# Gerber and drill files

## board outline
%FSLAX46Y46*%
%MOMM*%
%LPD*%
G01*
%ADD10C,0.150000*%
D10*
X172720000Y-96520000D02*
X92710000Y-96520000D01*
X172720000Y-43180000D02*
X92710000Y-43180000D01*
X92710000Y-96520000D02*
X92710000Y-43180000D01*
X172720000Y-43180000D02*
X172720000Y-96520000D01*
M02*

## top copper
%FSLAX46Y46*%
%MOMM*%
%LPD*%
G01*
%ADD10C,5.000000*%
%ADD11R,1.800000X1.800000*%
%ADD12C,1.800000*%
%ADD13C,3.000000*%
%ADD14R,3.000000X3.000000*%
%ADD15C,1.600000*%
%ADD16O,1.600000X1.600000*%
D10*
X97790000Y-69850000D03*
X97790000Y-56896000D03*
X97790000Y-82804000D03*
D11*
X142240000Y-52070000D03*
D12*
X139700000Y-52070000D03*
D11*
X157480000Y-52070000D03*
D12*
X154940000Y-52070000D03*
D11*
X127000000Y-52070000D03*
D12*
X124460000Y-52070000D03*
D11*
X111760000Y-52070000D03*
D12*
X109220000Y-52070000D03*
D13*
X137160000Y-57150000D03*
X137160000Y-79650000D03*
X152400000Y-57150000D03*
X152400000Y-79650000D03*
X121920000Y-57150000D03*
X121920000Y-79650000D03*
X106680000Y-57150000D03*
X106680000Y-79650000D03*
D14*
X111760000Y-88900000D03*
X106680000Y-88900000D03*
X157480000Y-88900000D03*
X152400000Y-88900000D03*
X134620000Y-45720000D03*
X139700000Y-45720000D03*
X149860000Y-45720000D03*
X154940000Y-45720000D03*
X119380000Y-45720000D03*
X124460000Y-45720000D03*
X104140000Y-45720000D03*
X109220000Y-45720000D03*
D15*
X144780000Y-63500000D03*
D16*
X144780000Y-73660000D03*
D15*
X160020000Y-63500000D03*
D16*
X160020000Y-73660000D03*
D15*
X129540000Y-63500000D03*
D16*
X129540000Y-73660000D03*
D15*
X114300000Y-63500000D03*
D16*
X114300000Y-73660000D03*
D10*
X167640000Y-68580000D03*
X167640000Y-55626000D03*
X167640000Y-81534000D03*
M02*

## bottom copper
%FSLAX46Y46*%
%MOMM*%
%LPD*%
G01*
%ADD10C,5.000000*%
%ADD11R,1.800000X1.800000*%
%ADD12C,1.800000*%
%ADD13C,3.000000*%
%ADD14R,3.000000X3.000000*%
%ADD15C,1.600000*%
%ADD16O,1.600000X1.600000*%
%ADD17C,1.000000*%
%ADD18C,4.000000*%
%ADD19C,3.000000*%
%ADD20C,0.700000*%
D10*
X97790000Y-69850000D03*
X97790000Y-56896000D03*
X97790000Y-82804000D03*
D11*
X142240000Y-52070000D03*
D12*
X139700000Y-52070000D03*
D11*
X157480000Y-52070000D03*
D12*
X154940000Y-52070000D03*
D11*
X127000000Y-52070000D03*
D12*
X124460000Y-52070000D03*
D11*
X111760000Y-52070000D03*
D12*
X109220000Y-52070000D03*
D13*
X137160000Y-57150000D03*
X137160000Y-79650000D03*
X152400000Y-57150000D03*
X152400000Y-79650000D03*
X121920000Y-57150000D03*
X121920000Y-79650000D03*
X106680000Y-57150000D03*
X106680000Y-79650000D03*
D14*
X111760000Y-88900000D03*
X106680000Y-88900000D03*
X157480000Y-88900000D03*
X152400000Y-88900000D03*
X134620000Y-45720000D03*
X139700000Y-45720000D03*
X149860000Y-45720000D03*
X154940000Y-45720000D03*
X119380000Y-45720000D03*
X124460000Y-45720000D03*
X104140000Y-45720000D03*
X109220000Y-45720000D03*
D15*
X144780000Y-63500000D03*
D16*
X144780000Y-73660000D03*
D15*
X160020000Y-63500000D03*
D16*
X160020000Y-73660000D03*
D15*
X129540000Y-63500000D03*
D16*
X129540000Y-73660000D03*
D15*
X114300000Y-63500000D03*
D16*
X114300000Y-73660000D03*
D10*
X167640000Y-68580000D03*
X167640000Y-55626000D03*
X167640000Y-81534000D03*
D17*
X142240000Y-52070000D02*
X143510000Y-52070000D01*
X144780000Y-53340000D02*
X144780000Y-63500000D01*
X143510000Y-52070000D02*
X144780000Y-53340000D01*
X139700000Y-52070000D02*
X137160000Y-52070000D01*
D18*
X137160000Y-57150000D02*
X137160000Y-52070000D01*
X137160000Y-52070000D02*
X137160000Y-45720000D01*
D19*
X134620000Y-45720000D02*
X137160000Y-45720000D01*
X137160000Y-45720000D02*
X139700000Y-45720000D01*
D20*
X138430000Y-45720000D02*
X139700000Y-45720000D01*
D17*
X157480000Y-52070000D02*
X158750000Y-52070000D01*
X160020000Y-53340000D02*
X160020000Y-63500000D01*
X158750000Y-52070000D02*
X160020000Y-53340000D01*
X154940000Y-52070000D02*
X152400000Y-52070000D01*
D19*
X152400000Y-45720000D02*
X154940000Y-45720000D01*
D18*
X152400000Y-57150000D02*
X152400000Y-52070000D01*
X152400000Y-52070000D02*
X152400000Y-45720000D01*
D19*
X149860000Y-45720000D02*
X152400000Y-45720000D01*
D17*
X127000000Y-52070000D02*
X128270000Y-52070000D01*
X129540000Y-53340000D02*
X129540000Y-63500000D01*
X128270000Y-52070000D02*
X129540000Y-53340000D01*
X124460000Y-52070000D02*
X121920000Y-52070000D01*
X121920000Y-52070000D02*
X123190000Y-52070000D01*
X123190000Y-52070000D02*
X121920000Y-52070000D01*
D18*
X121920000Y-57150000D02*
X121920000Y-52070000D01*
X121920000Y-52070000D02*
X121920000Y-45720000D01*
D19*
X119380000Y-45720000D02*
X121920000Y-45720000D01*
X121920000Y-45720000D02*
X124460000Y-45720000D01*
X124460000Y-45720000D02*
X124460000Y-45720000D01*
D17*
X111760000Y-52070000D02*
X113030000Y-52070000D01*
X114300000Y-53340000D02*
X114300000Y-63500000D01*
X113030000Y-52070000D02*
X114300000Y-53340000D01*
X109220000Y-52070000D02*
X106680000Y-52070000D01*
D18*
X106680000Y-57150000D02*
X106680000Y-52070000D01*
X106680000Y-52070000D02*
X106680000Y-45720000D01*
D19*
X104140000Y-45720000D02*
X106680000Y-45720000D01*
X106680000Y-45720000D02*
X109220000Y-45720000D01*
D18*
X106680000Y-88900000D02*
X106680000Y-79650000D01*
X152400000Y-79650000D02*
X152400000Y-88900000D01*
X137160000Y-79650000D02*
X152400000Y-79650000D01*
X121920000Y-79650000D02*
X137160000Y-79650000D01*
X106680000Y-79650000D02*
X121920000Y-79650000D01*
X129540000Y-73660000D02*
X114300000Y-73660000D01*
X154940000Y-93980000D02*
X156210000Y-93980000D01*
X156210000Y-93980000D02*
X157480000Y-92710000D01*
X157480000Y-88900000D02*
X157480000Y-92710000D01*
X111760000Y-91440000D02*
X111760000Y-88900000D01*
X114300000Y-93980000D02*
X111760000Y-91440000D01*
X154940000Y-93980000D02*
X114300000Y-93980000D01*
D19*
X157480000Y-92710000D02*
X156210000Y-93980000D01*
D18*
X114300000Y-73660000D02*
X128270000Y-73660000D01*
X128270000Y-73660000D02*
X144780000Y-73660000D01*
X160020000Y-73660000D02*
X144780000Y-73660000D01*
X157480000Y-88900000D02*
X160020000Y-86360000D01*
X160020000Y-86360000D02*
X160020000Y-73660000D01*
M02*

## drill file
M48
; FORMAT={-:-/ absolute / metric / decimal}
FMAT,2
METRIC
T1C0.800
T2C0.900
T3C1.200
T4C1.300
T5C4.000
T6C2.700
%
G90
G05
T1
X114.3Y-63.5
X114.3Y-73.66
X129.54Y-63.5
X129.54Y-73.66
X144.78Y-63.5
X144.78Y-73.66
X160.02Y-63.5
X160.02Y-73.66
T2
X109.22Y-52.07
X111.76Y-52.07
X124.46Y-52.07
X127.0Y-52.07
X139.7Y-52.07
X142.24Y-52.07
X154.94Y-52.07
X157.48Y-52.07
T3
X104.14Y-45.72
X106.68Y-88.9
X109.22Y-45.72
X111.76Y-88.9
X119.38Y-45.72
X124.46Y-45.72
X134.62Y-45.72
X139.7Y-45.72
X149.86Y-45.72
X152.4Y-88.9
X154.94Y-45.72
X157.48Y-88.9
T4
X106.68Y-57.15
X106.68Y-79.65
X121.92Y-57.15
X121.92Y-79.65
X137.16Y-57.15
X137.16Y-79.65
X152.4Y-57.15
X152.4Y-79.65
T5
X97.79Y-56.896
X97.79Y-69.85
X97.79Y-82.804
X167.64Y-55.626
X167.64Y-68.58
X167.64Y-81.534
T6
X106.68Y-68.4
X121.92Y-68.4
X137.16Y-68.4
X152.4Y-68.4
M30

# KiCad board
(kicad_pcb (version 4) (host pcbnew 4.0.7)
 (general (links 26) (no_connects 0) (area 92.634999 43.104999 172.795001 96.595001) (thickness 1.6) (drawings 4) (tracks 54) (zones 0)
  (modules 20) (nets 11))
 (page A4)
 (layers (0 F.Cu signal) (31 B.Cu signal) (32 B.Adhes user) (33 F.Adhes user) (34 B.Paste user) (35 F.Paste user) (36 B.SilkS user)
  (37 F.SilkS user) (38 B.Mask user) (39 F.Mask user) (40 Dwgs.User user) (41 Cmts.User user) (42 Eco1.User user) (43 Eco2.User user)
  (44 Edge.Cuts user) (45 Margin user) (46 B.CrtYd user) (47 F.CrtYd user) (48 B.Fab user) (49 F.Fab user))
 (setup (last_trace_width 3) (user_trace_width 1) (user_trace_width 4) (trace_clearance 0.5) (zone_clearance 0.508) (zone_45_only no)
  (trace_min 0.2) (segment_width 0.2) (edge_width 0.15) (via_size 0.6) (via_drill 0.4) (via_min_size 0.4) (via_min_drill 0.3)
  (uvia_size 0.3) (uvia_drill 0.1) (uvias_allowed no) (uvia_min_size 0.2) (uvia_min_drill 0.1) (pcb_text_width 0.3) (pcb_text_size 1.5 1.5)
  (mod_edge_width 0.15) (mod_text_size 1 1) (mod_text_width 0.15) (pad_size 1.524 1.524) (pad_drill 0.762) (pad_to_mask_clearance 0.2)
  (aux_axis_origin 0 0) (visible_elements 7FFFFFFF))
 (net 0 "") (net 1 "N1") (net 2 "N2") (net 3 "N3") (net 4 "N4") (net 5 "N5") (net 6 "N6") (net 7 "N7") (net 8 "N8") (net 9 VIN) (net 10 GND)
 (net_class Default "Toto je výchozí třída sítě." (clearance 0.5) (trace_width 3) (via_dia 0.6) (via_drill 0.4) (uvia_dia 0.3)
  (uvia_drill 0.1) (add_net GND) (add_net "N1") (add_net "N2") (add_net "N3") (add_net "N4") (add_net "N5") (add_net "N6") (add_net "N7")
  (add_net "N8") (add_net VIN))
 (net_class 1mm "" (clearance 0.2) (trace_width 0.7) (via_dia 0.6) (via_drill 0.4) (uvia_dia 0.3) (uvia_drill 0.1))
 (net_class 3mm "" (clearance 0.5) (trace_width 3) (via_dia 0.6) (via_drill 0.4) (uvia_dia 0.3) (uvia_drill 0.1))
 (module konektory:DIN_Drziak (layer F.Cu) (at 97.79 69.85)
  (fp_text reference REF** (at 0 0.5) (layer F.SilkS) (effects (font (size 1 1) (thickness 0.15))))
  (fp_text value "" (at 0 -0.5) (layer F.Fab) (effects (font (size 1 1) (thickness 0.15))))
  (pad 1 thru_hole circle (at 0 0) (size 5 5) (drill 4) (layers *.Cu *.Mask))
  (pad 1 thru_hole circle (at 0 -12.954) (size 5 5) (drill 4) (layers *.Cu *.Mask))
  (pad 1 thru_hole circle (at 0 12.954) (size 5 5) (drill 4) (layers *.Cu *.Mask)))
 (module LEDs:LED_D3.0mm (layer F.Cu) (at 142.24 52.07 180)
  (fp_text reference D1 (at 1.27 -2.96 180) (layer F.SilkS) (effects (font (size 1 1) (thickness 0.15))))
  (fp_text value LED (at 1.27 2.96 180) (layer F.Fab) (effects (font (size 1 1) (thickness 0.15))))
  (pad 1 thru_hole rect (at 0 0 180) (size 1.8 1.8) (drill 0.9) (layers *.Cu *.Mask) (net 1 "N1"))
  (pad 2 thru_hole circle (at 2.54 0 180) (size 1.8 1.8) (drill 0.9) (layers *.Cu *.Mask) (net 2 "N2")))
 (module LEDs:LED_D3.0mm (layer F.Cu) (at 157.48 52.07 180)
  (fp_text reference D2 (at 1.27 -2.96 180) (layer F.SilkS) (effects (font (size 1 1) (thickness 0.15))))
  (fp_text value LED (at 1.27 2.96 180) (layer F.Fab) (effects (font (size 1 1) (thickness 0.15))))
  (pad 1 thru_hole rect (at 0 0 180) (size 1.8 1.8) (drill 0.9) (layers *.Cu *.Mask) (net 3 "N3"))
  (pad 2 thru_hole circle (at 2.54 0 180) (size 1.8 1.8) (drill 0.9) (layers *.Cu *.Mask) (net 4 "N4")))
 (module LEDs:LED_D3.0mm (layer F.Cu) (at 127 52.07 180)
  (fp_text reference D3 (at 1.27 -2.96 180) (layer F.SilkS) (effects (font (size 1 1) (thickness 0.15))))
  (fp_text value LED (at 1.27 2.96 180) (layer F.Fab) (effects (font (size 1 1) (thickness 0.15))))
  (pad 1 thru_hole rect (at 0 0 180) (size 1.8 1.8) (drill 0.9) (layers *.Cu *.Mask) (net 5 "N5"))
  (pad 2 thru_hole circle (at 2.54 0 180) (size 1.8 1.8) (drill 0.9) (layers *.Cu *.Mask) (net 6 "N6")))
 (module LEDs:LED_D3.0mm (layer F.Cu) (at 111.76 52.07 180)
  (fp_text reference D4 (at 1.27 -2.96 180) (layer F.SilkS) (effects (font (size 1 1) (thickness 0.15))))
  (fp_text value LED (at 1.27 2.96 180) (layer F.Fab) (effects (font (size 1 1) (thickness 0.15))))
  (pad 1 thru_hole rect (at 0 0 180) (size 1.8 1.8) (drill 0.9) (layers *.Cu *.Mask) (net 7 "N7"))
  (pad 2 thru_hole circle (at 2.54 0 180) (size 1.8 1.8) (drill 0.9) (layers *.Cu *.Mask) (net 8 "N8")))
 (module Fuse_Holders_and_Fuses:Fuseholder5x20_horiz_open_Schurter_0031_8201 (layer F.Cu) (at 137.16 57.15 270)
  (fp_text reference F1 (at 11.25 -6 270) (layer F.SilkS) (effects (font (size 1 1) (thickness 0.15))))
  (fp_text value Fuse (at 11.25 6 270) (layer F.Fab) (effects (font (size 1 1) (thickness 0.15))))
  (pad 1 thru_hole circle (at 0 0 270) (size 3 3) (drill 1.3) (layers *.Cu *.Mask) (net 2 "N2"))
  (pad 2 thru_hole circle (at 22.5 0 270) (size 3 3) (drill 1.3) (layers *.Cu *.Mask) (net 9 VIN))
  (pad "" np_thru_hole circle (at 11.25 0 270) (size 2.7 2.7) (drill 2.7) (layers *.Cu *.Mask)))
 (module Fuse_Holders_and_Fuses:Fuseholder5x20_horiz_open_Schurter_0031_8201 (layer F.Cu) (at 152.4 57.15 270)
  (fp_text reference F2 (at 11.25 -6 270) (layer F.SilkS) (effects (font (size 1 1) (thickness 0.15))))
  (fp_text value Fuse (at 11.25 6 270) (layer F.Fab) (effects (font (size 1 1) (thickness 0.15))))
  (pad 1 thru_hole circle (at 0 0 270) (size 3 3) (drill 1.3) (layers *.Cu *.Mask) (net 4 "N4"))
  (pad 2 thru_hole circle (at 22.5 0 270) (size 3 3) (drill 1.3) (layers *.Cu *.Mask) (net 9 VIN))
  (pad "" np_thru_hole circle (at 11.25 0 270) (size 2.7 2.7) (drill 2.7) (layers *.Cu *.Mask)))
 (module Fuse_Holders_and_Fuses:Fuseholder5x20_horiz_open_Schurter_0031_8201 (layer F.Cu) (at 121.92 57.15 270)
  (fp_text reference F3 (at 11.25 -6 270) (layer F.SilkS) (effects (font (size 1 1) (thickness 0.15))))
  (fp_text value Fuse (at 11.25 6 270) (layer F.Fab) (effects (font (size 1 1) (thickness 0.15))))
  (pad 1 thru_hole circle (at 0 0 270) (size 3 3) (drill 1.3) (layers *.Cu *.Mask) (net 6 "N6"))
  (pad 2 thru_hole circle (at 22.5 0 270) (size 3 3) (drill 1.3) (layers *.Cu *.Mask) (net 9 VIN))
  (pad "" np_thru_hole circle (at 11.25 0 270) (size 2.7 2.7) (drill 2.7) (layers *.Cu *.Mask)))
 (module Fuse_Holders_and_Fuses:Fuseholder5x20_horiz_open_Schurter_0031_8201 (layer F.Cu) (at 106.68 57.15 270)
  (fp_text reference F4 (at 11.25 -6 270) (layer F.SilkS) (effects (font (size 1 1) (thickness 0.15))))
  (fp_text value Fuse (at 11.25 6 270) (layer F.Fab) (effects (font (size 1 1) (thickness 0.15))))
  (pad 1 thru_hole circle (at 0 0 270) (size 3 3) (drill 1.3) (layers *.Cu *.Mask) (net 8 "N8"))
  (pad 2 thru_hole circle (at 22.5 0 270) (size 3 3) (drill 1.3) (layers *.Cu *.Mask) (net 9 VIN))
  (pad "" np_thru_hole circle (at 11.25 0 270) (size 2.7 2.7) (drill 2.7) (layers *.Cu *.Mask)))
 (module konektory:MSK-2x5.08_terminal (layer F.Cu) (at 109.22 88.9 180)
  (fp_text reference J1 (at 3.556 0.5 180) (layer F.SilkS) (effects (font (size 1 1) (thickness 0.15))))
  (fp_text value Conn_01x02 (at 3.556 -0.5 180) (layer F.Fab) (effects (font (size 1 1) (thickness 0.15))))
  (pad 1 thru_hole rect (at -2.54 0 180) (size 3 3) (drill 1.2) (layers *.Mask B.Cu) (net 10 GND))
  (pad 2 thru_hole rect (at 2.54 0 180) (size 3 3) (drill 1.2) (layers *.Mask B.Cu) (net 9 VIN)))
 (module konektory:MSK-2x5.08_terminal (layer F.Cu) (at 154.94 88.9 180)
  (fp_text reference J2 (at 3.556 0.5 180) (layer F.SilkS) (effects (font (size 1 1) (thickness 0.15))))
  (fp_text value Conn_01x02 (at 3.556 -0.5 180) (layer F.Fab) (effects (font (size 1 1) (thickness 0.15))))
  (pad 1 thru_hole rect (at -2.54 0 180) (size 3 3) (drill 1.2) (layers *.Mask B.Cu) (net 10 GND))
  (pad 2 thru_hole rect (at 2.54 0 180) (size 3 3) (drill 1.2) (layers *.Mask B.Cu) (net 9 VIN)))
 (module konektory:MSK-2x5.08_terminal (layer F.Cu) (at 137.16 45.72)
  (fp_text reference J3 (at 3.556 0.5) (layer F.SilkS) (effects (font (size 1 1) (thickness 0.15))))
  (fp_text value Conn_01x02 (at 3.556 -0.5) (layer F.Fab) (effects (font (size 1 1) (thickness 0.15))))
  (pad 1 thru_hole rect (at -2.54 0) (size 3 3) (drill 1.2) (layers *.Mask B.Cu) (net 2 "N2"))
  (pad 2 thru_hole rect (at 2.54 0) (size 3 3) (drill 1.2) (layers *.Mask B.Cu) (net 2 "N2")))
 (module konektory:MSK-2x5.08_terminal (layer F.Cu) (at 152.4 45.72)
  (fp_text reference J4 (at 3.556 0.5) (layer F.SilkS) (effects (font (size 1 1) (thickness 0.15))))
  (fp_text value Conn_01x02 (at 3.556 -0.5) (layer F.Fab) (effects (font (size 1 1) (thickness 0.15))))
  (pad 1 thru_hole rect (at -2.54 0) (size 3 3) (drill 1.2) (layers *.Mask B.Cu) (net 4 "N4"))
  (pad 2 thru_hole rect (at 2.54 0) (size 3 3) (drill 1.2) (layers *.Mask B.Cu) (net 4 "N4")))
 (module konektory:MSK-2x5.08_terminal (layer F.Cu) (at 121.92 45.72)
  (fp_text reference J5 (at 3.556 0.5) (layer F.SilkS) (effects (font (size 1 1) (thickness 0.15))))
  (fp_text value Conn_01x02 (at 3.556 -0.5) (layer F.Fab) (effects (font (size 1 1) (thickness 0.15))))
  (pad 1 thru_hole rect (at -2.54 0) (size 3 3) (drill 1.2) (layers *.Mask B.Cu) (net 6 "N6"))
  (pad 2 thru_hole rect (at 2.54 0) (size 3 3) (drill 1.2) (layers *.Mask B.Cu) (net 6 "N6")))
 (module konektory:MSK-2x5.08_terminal (layer F.Cu) (at 106.68 45.72)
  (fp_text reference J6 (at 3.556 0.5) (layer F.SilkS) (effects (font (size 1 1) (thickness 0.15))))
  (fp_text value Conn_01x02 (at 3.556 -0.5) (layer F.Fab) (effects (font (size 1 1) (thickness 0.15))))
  (pad 1 thru_hole rect (at -2.54 0) (size 3 3) (drill 1.2) (layers *.Mask B.Cu) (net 8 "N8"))
  (pad 2 thru_hole rect (at 2.54 0) (size 3 3) (drill 1.2) (layers *.Mask B.Cu) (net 8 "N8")))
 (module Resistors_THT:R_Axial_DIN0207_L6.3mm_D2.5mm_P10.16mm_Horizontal (layer F.Cu) (at 144.78 63.5 270)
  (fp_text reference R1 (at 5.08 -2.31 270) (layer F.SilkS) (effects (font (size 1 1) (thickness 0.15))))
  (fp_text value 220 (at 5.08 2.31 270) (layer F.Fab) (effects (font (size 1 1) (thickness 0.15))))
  (pad 1 thru_hole circle (at 0 0 270) (size 1.6 1.6) (drill 0.8) (layers *.Cu *.Mask) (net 1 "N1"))
  (pad 2 thru_hole oval (at 10.16 0 270) (size 1.6 1.6) (drill 0.8) (layers *.Cu *.Mask) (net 10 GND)))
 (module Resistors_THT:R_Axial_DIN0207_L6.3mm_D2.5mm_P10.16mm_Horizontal (layer F.Cu) (at 160.02 63.5 270)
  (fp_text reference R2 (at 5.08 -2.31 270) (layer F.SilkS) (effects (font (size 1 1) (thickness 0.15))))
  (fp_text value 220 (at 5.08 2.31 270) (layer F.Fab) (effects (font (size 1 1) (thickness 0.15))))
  (pad 1 thru_hole circle (at 0 0 270) (size 1.6 1.6) (drill 0.8) (layers *.Cu *.Mask) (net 3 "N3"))
  (pad 2 thru_hole oval (at 10.16 0 270) (size 1.6 1.6) (drill 0.8) (layers *.Cu *.Mask) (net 10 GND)))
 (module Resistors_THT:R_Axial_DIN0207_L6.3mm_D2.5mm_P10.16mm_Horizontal (layer F.Cu) (at 129.54 63.5 270)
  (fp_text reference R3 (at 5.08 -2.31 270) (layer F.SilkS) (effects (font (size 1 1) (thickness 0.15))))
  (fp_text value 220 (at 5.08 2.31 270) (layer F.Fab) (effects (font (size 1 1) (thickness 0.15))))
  (pad 1 thru_hole circle (at 0 0 270) (size 1.6 1.6) (drill 0.8) (layers *.Cu *.Mask) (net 5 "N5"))
  (pad 2 thru_hole oval (at 10.16 0 270) (size 1.6 1.6) (drill 0.8) (layers *.Cu *.Mask) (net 10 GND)))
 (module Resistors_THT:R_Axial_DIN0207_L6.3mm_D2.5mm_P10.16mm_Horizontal (layer F.Cu) (at 114.3 63.5 270)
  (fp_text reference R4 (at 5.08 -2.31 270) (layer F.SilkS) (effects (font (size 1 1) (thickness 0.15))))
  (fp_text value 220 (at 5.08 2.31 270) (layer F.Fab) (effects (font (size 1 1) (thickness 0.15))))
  (pad 1 thru_hole circle (at 0 0 270) (size 1.6 1.6) (drill 0.8) (layers *.Cu *.Mask) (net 7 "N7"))
  (pad 2 thru_hole oval (at 10.16 0 270) (size 1.6 1.6) (drill 0.8) (layers *.Cu *.Mask) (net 10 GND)))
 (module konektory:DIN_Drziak (layer F.Cu) (at 167.64 68.58)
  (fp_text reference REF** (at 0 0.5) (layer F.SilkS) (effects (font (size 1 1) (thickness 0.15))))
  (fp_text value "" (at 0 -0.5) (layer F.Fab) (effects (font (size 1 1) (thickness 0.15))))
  (pad 1 thru_hole circle (at 0 0) (size 5 5) (drill 4) (layers *.Cu *.Mask))
  (pad 1 thru_hole circle (at 0 -12.954) (size 5 5) (drill 4) (layers *.Cu *.Mask))
  (pad 1 thru_hole circle (at 0 12.954) (size 5 5) (drill 4) (layers *.Cu *.Mask)))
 (gr_line (start 172.72 96.52) (end 92.71 96.52) (angle 90) (layer Edge.Cuts) (width 0.15))
 (gr_line (start 172.72 43.18) (end 92.71 43.18) (angle 90) (layer Edge.Cuts) (width 0.15))
 (gr_line (start 92.71 96.52) (end 92.71 43.18) (angle 90) (layer Edge.Cuts) (width 0.15))
 (gr_line (start 172.72 43.18) (end 172.72 96.52) (angle 90) (layer Edge.Cuts) (width 0.15))
 (segment (start 142.24 52.07) (end 143.51 52.07) (width 1) (layer B.Cu) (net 1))
 (segment (start 144.78 53.34) (end 144.78 63.5) (width 1) (layer B.Cu) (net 1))
 (segment (start 143.51 52.07) (end 144.78 53.34) (width 1) (layer B.Cu) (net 1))
 (segment (start 139.7 52.07) (end 137.16 52.07) (width 1) (layer B.Cu) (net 2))
 (segment (start 137.16 57.15) (end 137.16 52.07) (width 4) (layer B.Cu) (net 2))
 (segment (start 137.16 52.07) (end 137.16 45.72) (width 4) (layer B.Cu) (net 2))
 (segment (start 134.62 45.72) (end 137.16 45.72) (width 3) (layer B.Cu) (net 2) (status 30))
 (segment (start 137.16 45.72) (end 139.7 45.72) (width 3) (layer B.Cu) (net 2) (status 30))
 (segment (start 138.43 45.72) (end 139.7 45.72) (width 0.7) (layer B.Cu) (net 2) (status 30))
 (segment (start 157.48 52.07) (end 158.75 52.07) (width 1) (layer B.Cu) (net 3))
 (segment (start 160.02 53.34) (end 160.02 63.5) (width 1) (layer B.Cu) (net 3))
 (segment (start 158.75 52.07) (end 160.02 53.34) (width 1) (layer B.Cu) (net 3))
 (segment (start 154.94 52.07) (end 152.4 52.07) (width 1) (layer B.Cu) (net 4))
 (segment (start 152.4 45.72) (end 154.94 45.72) (width 3) (layer B.Cu) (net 4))
 (segment (start 152.4 57.15) (end 152.4 52.07) (width 4) (layer B.Cu) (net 4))
 (segment (start 152.4 52.07) (end 152.4 45.72) (width 4) (layer B.Cu) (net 4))
 (segment (start 149.86 45.72) (end 152.4 45.72) (width 3) (layer B.Cu) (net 4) (status 10))
 (segment (start 127 52.07) (end 128.27 52.07) (width 1) (layer B.Cu) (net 5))
 (segment (start 129.54 53.34) (end 129.54 63.5) (width 1) (layer B.Cu) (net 5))
 (segment (start 128.27 52.07) (end 129.54 53.34) (width 1) (layer B.Cu) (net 5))
 (segment (start 124.46 52.07) (end 121.92 52.07) (width 1) (layer B.Cu) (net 6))
 (segment (start 121.92 52.07) (end 123.19 52.07) (width 1) (layer B.Cu) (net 6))
 (segment (start 123.19 52.07) (end 121.92 52.07) (width 1) (layer B.Cu) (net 6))
 (segment (start 121.92 57.15) (end 121.92 52.07) (width 4) (layer B.Cu) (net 6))
 (segment (start 121.92 52.07) (end 121.92 45.72) (width 4) (layer B.Cu) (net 6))
 (segment (start 119.38 45.72) (end 121.92 45.72) (width 3) (layer B.Cu) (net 6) (status 10))
 (segment (start 121.92 45.72) (end 124.46 45.72) (width 3) (layer B.Cu) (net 6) (status 10))
 (segment (start 124.46 45.72) (end 124.46 45.72) (width 3) (layer B.Cu) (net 6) (status 20))
 (segment (start 111.76 52.07) (end 113.03 52.07) (width 1) (layer B.Cu) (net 7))
 (segment (start 114.3 53.34) (end 114.3 63.5) (width 1) (layer B.Cu) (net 7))
 (segment (start 113.03 52.07) (end 114.3 53.34) (width 1) (layer B.Cu) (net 7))
 (segment (start 109.22 52.07) (end 106.68 52.07) (width 1) (layer B.Cu) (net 8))
 (segment (start 106.68 57.15) (end 106.68 52.07) (width 4) (layer B.Cu) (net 8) (status 10))
 (segment (start 106.68 52.07) (end 106.68 45.72) (width 4) (layer B.Cu) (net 8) (status 10))
 (segment (start 104.14 45.72) (end 106.68 45.72) (width 3) (layer B.Cu) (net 8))
 (segment (start 106.68 45.72) (end 109.22 45.72) (width 3) (layer B.Cu) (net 8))
 (segment (start 106.68 88.9) (end 106.68 79.65) (width 4) (layer B.Cu) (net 9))
 (segment (start 152.4 79.65) (end 152.4 88.9) (width 4) (layer B.Cu) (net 9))
 (segment (start 137.16 79.65) (end 152.4 79.65) (width 4) (layer B.Cu) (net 9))
 (segment (start 121.92 79.65) (end 137.16 79.65) (width 4) (layer B.Cu) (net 9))
 (segment (start 106.68 79.65) (end 121.92 79.65) (width 4) (layer B.Cu) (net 9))
 (segment (start 129.54 73.66) (end 114.3 73.66) (width 4) (layer B.Cu) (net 10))
 (segment (start 154.94 93.98) (end 156.21 93.98) (width 4) (layer B.Cu) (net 10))
 (segment (start 156.21 93.98) (end 157.48 92.71) (width 4) (layer B.Cu) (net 10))
 (segment (start 157.48 88.9) (end 157.48 92.71) (width 4) (layer B.Cu) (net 10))
 (segment (start 111.76 91.44) (end 111.76 88.9) (width 4) (layer B.Cu) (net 10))
 (segment (start 114.3 93.98) (end 111.76 91.44) (width 4) (layer B.Cu) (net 10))
 (segment (start 154.94 93.98) (end 114.3 93.98) (width 4) (layer B.Cu) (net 10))
 (segment (start 157.48 92.71) (end 156.21 93.98) (width 3) (layer B.Cu) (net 10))
 (segment (start 114.3 73.66) (end 128.27 73.66) (width 4) (layer B.Cu) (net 10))
 (segment (start 128.27 73.66) (end 144.78 73.66) (width 4) (layer B.Cu) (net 10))
 (segment (start 160.02 73.66) (end 144.78 73.66) (width 4) (layer B.Cu) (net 10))
 (segment (start 157.48 88.9) (end 160.02 86.36) (width 4) (layer B.Cu) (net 10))
 (segment (start 160.02 86.36) (end 160.02 73.66) (width 4) (layer B.Cu) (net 10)))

